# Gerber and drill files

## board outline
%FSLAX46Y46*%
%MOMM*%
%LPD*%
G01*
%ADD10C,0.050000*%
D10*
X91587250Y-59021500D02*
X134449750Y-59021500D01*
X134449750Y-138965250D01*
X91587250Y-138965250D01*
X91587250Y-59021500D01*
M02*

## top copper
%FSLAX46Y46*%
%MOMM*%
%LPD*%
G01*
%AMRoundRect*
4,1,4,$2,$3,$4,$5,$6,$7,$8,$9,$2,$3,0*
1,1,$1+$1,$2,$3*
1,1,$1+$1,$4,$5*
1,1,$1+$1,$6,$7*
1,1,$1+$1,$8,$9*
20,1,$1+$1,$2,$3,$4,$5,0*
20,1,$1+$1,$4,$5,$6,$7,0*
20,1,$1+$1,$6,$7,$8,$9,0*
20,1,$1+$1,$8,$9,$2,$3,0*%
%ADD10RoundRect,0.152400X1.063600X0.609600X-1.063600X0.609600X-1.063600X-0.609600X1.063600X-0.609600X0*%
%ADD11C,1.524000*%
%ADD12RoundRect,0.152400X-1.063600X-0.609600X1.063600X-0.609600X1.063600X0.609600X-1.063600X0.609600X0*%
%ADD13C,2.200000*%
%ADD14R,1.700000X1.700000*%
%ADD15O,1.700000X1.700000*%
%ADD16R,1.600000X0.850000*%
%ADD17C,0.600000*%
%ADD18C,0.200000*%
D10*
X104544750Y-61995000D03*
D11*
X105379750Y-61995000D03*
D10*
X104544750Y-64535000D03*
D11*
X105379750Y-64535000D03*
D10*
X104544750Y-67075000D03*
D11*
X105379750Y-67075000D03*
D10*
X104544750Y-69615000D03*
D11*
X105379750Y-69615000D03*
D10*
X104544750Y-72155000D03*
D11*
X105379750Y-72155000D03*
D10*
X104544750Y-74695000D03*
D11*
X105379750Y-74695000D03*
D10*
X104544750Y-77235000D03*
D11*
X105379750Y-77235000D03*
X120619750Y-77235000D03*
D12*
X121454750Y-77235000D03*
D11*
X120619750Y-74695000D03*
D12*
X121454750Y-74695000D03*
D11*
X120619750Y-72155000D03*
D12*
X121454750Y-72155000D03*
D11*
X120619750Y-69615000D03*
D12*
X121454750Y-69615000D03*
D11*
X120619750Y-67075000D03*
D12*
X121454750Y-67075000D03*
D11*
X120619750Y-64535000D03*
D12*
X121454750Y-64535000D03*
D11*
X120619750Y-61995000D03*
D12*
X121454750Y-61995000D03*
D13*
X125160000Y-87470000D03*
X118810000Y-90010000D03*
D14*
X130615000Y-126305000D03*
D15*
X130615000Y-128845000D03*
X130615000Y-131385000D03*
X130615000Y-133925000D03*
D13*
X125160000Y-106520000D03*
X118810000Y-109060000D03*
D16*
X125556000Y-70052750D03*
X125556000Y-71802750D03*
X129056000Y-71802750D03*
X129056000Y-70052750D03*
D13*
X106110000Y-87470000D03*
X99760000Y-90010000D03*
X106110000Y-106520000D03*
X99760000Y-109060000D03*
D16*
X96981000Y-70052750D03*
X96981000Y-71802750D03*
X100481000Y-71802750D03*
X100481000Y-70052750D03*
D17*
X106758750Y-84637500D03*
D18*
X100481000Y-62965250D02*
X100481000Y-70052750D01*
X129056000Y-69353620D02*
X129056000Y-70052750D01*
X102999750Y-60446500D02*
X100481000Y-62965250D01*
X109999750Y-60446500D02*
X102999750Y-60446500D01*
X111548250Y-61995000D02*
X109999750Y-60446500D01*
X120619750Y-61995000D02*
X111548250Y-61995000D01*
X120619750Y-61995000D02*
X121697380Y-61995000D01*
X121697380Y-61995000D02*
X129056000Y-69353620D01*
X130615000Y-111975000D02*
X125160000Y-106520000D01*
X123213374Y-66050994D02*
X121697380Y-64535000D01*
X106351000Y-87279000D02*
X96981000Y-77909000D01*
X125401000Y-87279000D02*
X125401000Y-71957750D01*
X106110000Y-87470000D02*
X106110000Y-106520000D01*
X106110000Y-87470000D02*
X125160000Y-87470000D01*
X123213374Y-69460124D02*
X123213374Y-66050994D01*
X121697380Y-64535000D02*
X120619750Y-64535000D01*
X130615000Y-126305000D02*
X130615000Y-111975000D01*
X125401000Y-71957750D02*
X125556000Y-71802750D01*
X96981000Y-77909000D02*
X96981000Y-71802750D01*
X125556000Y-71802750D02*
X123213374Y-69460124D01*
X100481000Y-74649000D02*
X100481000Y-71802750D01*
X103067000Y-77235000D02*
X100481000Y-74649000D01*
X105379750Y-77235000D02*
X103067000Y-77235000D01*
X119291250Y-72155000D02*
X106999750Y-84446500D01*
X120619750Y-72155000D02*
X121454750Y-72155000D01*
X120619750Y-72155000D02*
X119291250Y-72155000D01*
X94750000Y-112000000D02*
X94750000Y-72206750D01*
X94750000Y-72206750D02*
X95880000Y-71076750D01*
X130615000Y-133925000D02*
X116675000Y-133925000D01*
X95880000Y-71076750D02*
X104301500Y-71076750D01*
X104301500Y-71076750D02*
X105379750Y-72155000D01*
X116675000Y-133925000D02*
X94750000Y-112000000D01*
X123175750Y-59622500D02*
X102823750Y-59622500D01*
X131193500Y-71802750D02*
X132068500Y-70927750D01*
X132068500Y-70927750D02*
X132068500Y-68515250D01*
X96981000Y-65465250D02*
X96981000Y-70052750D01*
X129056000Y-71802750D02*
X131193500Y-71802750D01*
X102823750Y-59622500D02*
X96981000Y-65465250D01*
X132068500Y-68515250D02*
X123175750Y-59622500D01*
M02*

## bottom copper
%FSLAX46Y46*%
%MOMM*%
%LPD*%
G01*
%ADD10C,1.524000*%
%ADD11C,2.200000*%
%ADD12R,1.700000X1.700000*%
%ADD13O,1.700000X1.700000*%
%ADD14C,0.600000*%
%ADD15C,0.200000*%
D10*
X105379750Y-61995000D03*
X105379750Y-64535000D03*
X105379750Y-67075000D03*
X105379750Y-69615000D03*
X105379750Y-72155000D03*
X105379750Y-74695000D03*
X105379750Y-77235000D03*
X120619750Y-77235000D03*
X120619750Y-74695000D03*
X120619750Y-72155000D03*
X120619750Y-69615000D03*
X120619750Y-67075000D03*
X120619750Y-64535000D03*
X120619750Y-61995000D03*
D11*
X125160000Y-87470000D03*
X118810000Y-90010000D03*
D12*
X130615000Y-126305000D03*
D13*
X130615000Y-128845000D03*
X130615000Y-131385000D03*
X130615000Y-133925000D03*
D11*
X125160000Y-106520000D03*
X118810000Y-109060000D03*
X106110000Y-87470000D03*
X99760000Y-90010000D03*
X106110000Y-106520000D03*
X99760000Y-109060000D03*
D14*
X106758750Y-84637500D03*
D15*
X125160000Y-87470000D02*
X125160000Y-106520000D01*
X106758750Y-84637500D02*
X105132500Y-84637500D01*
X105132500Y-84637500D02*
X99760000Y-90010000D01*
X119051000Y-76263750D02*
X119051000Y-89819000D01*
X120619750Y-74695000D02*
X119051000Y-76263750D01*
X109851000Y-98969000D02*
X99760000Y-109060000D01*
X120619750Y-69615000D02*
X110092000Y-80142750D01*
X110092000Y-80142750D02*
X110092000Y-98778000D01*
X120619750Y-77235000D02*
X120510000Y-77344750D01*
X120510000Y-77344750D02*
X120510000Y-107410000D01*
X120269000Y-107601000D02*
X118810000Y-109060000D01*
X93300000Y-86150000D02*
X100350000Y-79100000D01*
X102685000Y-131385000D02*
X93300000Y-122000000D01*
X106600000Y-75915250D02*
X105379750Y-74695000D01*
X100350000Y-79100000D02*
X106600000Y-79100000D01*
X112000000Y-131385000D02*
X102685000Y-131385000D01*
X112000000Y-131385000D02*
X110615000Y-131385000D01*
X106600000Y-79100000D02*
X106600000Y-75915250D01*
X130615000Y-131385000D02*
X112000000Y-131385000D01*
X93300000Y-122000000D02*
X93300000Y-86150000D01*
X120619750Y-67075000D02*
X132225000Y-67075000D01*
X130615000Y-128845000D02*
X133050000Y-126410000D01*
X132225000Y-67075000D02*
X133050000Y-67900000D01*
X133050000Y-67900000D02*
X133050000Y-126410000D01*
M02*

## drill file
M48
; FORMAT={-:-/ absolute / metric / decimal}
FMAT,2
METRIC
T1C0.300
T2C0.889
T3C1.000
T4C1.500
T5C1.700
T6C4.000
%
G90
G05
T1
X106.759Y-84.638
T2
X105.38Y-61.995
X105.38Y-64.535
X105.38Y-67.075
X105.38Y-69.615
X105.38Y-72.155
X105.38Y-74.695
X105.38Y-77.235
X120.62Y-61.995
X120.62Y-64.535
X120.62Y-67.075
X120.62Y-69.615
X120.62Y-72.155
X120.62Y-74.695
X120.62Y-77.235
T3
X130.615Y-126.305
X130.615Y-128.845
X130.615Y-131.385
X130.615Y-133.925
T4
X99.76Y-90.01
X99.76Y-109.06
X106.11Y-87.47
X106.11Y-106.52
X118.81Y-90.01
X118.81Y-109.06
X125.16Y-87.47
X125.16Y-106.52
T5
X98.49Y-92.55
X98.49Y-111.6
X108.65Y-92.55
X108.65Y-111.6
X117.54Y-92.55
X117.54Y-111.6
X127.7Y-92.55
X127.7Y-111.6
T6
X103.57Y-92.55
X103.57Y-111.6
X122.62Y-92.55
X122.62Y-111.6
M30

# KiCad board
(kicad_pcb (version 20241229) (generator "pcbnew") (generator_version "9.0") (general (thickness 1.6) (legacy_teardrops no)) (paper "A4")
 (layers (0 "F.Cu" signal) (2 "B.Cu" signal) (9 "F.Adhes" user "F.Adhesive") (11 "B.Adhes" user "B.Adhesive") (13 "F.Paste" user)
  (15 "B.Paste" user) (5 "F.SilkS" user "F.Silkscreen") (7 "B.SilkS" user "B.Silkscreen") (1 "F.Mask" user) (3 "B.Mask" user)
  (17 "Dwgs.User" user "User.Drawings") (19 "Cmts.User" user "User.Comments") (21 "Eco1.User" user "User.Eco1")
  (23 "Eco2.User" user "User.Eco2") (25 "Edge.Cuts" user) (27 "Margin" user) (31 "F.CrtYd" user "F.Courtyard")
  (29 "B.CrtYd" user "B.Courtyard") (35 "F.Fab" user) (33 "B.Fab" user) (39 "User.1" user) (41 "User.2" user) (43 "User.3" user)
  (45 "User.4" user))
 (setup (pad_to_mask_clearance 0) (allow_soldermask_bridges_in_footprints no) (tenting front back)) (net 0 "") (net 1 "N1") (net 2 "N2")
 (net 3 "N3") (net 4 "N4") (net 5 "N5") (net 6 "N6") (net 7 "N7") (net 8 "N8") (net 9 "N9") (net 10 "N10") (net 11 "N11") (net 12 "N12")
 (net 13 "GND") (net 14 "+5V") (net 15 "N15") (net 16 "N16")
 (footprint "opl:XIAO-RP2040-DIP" (layer "F.Cu") (at 112.99975 69.615)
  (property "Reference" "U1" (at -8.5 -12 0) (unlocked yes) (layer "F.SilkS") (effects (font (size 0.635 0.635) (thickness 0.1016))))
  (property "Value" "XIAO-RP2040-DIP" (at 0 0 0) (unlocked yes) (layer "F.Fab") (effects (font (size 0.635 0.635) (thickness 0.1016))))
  (pad "1" smd roundrect (at -8.455 -7.62 180) (size 2.432 1.524) (layers "F.Cu" "F.Mask") (roundrect_rratio 0.1) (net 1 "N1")
   (thermal_bridge_angle 45))
  (pad "1" thru_hole circle (at -7.62 -7.62 180) (size 1.524 1.524) (drill 0.889) (layers "*.Cu" "*.Mask") (remove_unused_layers no)
   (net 1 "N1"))
  (pad "2" smd roundrect (at -8.455 -5.08 180) (size 2.432 1.524) (layers "F.Cu" "F.Mask") (roundrect_rratio 0.1) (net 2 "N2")
   (thermal_bridge_angle 45))
  (pad "2" thru_hole circle (at -7.62 -5.08 180) (size 1.524 1.524) (drill 0.889) (layers "*.Cu" "*.Mask") (remove_unused_layers no)
   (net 2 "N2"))
  (pad "3" smd roundrect (at -8.455 -2.54 180) (size 2.432 1.524) (layers "F.Cu" "F.Mask") (roundrect_rratio 0.1) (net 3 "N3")
   (thermal_bridge_angle 45))
  (pad "3" thru_hole circle (at -7.62 -2.54 180) (size 1.524 1.524) (drill 0.889) (layers "*.Cu" "*.Mask") (remove_unused_layers no)
   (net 3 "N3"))
  (pad "4" smd roundrect (at -8.455 0 180) (size 2.432 1.524) (layers "F.Cu" "F.Mask") (roundrect_rratio 0.1) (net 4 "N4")
   (thermal_bridge_angle 45))
  (pad "4" thru_hole circle (at -7.62 0 180) (size 1.524 1.524) (drill 0.889) (layers "*.Cu" "*.Mask") (remove_unused_layers no)
   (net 4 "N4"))
  (pad "5" smd roundrect (at -8.455 2.54 180) (size 2.432 1.524) (layers "F.Cu" "F.Mask") (roundrect_rratio 0.1) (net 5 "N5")
   (thermal_bridge_angle 45))
  (pad "5" thru_hole circle (at -7.62 2.54 180) (size 1.524 1.524) (drill 0.889) (layers "*.Cu" "*.Mask") (remove_unused_layers no)
   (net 5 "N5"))
  (pad "6" smd roundrect (at -8.455 5.08 180) (size 2.432 1.524) (layers "F.Cu" "F.Mask") (roundrect_rratio 0.1) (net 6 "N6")
   (thermal_bridge_angle 45))
  (pad "6" thru_hole circle (at -7.62 5.08 180) (size 1.524 1.524) (drill 0.889) (layers "*.Cu" "*.Mask") (remove_unused_layers no)
   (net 6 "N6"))
  (pad "7" smd roundrect (at -8.455 7.62 180) (size 2.432 1.524) (layers "F.Cu" "F.Mask") (roundrect_rratio 0.1) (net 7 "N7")
   (thermal_bridge_angle 45))
  (pad "7" thru_hole circle (at -7.62 7.62 180) (size 1.524 1.524) (drill 0.889) (layers "*.Cu" "*.Mask") (remove_unused_layers no)
   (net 7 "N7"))
  (pad "8" thru_hole circle (at 7.62 7.62) (size 1.524 1.524) (drill 0.889) (layers "*.Cu" "*.Mask") (remove_unused_layers no) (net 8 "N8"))
  (pad "8" smd roundrect (at 8.455 7.62) (size 2.432 1.524) (layers "F.Cu" "F.Mask") (roundrect_rratio 0.1) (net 8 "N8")
   (thermal_bridge_angle 45))
  (pad "9" thru_hole circle (at 7.62 5.08) (size 1.524 1.524) (drill 0.889) (layers "*.Cu" "*.Mask") (remove_unused_layers no) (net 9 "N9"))
  (pad "9" smd roundrect (at 8.455 5.08) (size 2.432 1.524) (layers "F.Cu" "F.Mask") (roundrect_rratio 0.1) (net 9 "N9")
   (thermal_bridge_angle 45))
  (pad "10" thru_hole circle (at 7.62 2.54) (size 1.524 1.524) (drill 0.889) (layers "*.Cu" "*.Mask") (remove_unused_layers no)
   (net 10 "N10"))
  (pad "10" smd roundrect (at 8.455 2.54) (size 2.432 1.524) (layers "F.Cu" "F.Mask") (roundrect_rratio 0.1) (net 10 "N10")
   (thermal_bridge_angle 45))
  (pad "11" thru_hole circle (at 7.62 0) (size 1.524 1.524) (drill 0.889) (layers "*.Cu" "*.Mask") (remove_unused_layers no) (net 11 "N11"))
  (pad "11" smd roundrect (at 8.455 0) (size 2.432 1.524) (layers "F.Cu" "F.Mask") (roundrect_rratio 0.1) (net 11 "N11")
   (thermal_bridge_angle 45))
  (pad "12" thru_hole circle (at 7.62 -2.54) (size 1.524 1.524) (drill 0.889) (layers "*.Cu" "*.Mask") (remove_unused_layers no)
   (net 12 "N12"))
  (pad "12" smd roundrect (at 8.455 -2.54) (size 2.432 1.524) (layers "F.Cu" "F.Mask") (roundrect_rratio 0.1) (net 12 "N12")
   (thermal_bridge_angle 45))
  (pad "13" thru_hole circle (at 7.62 -5.08) (size 1.524 1.524) (drill 0.889) (layers "*.Cu" "*.Mask") (remove_unused_layers no)
   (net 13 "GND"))
  (pad "13" smd roundrect (at 8.455 -5.08) (size 2.432 1.524) (layers "F.Cu" "F.Mask") (roundrect_rratio 0.1) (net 13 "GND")
   (thermal_bridge_angle 45))
  (pad "14" thru_hole circle (at 7.62 -7.62) (size 1.524 1.524) (drill 0.889) (layers "*.Cu" "*.Mask") (remove_unused_layers no)
   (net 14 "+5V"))
  (pad "14" smd roundrect (at 8.455 -7.62) (size 2.432 1.524) (layers "F.Cu" "F.Mask") (roundrect_rratio 0.1) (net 14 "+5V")
   (thermal_bridge_angle 45)))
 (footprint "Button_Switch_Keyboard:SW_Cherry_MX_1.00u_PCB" (layer "F.Cu") (at 125.16 87.47)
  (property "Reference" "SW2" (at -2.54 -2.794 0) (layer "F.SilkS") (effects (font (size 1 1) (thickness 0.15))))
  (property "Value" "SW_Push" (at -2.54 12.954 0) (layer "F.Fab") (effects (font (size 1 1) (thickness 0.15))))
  (pad "" np_thru_hole circle (at -7.62 5.08) (size 1.7 1.7) (drill 1.7) (layers "*.Cu" "*.Mask"))
  (pad "" np_thru_hole circle (at -2.54 5.08) (size 4 4) (drill 4) (layers "*.Cu" "*.Mask"))
  (pad "" np_thru_hole circle (at 2.54 5.08) (size 1.7 1.7) (drill 1.7) (layers "*.Cu" "*.Mask"))
  (pad "1" thru_hole circle (at 0 0) (size 2.2 2.2) (drill 1.5) (layers "*.Cu" "*.Mask") (remove_unused_layers no) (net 13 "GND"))
  (pad "2" thru_hole circle (at -6.35 2.54) (size 2.2 2.2) (drill 1.5) (layers "*.Cu" "*.Mask") (remove_unused_layers no) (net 9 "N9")))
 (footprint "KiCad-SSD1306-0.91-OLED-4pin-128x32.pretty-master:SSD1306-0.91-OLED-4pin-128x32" (layer "F.Cu") (at 94.115 124.115)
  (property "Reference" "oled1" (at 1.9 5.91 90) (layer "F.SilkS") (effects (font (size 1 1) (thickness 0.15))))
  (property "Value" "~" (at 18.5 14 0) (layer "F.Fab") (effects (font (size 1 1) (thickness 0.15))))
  (pad "1" thru_hole rect (at 36.5 2.19) (size 1.7 1.7) (drill 1) (layers "*.Cu" "*.Mask") (remove_unused_layers no) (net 13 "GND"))
  (pad "2" thru_hole oval (at 36.5 4.73) (size 1.7 1.7) (drill 1) (layers "*.Cu" "*.Mask") (remove_unused_layers no) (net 12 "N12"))
  (pad "3" thru_hole oval (at 36.5 7.27) (size 1.7 1.7) (drill 1) (layers "*.Cu" "*.Mask") (remove_unused_layers no) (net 6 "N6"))
  (pad "4" thru_hole oval (at 36.5 9.81) (size 1.7 1.7) (drill 1) (layers "*.Cu" "*.Mask") (remove_unused_layers no) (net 5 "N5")))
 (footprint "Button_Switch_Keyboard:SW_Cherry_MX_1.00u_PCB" (layer "F.Cu") (at 125.16 106.52)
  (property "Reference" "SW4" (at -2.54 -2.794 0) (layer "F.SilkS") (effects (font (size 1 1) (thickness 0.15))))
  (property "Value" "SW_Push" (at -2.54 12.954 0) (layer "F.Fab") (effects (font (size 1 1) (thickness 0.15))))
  (pad "" np_thru_hole circle (at -7.62 5.08) (size 1.7 1.7) (drill 1.7) (layers "*.Cu" "*.Mask"))
  (pad "" np_thru_hole circle (at -2.54 5.08) (size 4 4) (drill 4) (layers "*.Cu" "*.Mask"))
  (pad "" np_thru_hole circle (at 2.54 5.08) (size 1.7 1.7) (drill 1.7) (layers "*.Cu" "*.Mask"))
  (pad "1" thru_hole circle (at 0 0) (size 2.2 2.2) (drill 1.5) (layers "*.Cu" "*.Mask") (remove_unused_layers no) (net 13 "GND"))
  (pad "2" thru_hole circle (at -6.35 2.54) (size 2.2 2.2) (drill 1.5) (layers "*.Cu" "*.Mask") (remove_unused_layers no) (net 8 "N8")))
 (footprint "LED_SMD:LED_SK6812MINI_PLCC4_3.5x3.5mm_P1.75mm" (layer "F.Cu") (at 127.306 70.92775)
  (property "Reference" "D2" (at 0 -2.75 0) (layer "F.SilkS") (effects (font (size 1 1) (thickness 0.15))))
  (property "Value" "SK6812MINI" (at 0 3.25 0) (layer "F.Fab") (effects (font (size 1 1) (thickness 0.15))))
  (pad "1" smd rect (at -1.75 -0.875) (size 1.6 0.85) (layers "F.Cu" "F.Mask" "F.Paste") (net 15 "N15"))
  (pad "2" smd rect (at -1.75 0.875) (size 1.6 0.85) (layers "F.Cu" "F.Mask" "F.Paste") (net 13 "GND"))
  (pad "3" smd rect (at 1.75 0.875) (size 1.6 0.85) (layers "F.Cu" "F.Mask" "F.Paste") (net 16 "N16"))
  (pad "4" smd rect (at 1.75 -0.875) (size 1.6 0.85) (layers "F.Cu" "F.Mask" "F.Paste") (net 14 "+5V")))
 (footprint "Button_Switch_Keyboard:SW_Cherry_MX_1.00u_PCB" (layer "F.Cu") (at 106.11 87.47)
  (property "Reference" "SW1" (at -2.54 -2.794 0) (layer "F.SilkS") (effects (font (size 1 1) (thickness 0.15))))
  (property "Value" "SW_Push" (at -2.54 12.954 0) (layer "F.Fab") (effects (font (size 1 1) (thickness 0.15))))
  (pad "" np_thru_hole circle (at -7.62 5.08) (size 1.7 1.7) (drill 1.7) (layers "*.Cu" "*.Mask"))
  (pad "" np_thru_hole circle (at -2.54 5.08) (size 4 4) (drill 4) (layers "*.Cu" "*.Mask"))
  (pad "" np_thru_hole circle (at 2.54 5.08) (size 1.7 1.7) (drill 1.7) (layers "*.Cu" "*.Mask"))
  (pad "1" thru_hole circle (at 0 0) (size 2.2 2.2) (drill 1.5) (layers "*.Cu" "*.Mask") (remove_unused_layers no) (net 13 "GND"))
  (pad "2" thru_hole circle (at -6.35 2.54) (size 2.2 2.2) (drill 1.5) (layers "*.Cu" "*.Mask") (remove_unused_layers no) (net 10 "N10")))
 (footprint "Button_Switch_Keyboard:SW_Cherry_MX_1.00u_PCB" (layer "F.Cu") (at 106.11 106.52)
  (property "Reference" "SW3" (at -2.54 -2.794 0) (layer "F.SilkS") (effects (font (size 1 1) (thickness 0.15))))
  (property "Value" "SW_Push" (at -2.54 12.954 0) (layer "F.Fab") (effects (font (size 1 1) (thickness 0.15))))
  (pad "" np_thru_hole circle (at -7.62 5.08) (size 1.7 1.7) (drill 1.7) (layers "*.Cu" "*.Mask"))
  (pad "" np_thru_hole circle (at -2.54 5.08) (size 4 4) (drill 4) (layers "*.Cu" "*.Mask"))
  (pad "" np_thru_hole circle (at 2.54 5.08) (size 1.7 1.7) (drill 1.7) (layers "*.Cu" "*.Mask"))
  (pad "1" thru_hole circle (at 0 0) (size 2.2 2.2) (drill 1.5) (layers "*.Cu" "*.Mask") (remove_unused_layers no) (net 13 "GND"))
  (pad "2" thru_hole circle (at -6.35 2.54) (size 2.2 2.2) (drill 1.5) (layers "*.Cu" "*.Mask") (remove_unused_layers no) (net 11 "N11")))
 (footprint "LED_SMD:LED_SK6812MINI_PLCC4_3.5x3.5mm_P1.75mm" (layer "F.Cu") (at 98.731 70.92775)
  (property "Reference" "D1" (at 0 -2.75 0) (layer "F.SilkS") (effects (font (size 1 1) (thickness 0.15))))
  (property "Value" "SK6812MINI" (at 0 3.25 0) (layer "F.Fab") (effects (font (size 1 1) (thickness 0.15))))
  (pad "1" smd rect (at -1.75 -0.875) (size 1.6 0.85) (layers "F.Cu" "F.Mask" "F.Paste") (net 16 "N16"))
  (pad "2" smd rect (at -1.75 0.875) (size 1.6 0.85) (layers "F.Cu" "F.Mask" "F.Paste") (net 13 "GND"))
  (pad "3" smd rect (at 1.75 0.875) (size 1.6 0.85) (layers "F.Cu" "F.Mask" "F.Paste") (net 7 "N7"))
  (pad "4" smd rect (at 1.75 -0.875) (size 1.6 0.85) (layers "F.Cu" "F.Mask" "F.Paste") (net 14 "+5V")))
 (gr_rect (start 91.58725 59.0215) (end 134.44975 138.96525) (stroke (width 0.05) (type default)) (fill no) (layer "Edge.Cuts"))
 (segment (start 100.481 62.96525) (end 100.481 70.05275) (width 0.2) (layer "F.Cu") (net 14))
 (segment (start 129.056 69.35362) (end 129.056 70.05275) (width 0.2) (layer "F.Cu") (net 14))
 (segment (start 102.99975 60.4465) (end 100.481 62.96525) (width 0.2) (layer "F.Cu") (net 14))
 (segment (start 109.99975 60.4465) (end 102.99975 60.4465) (width 0.2) (layer "F.Cu") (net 14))
 (segment (start 111.54825 61.995) (end 109.99975 60.4465) (width 0.2) (layer "F.Cu") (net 14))
 (segment (start 120.61975 61.995) (end 111.54825 61.995) (width 0.2) (layer "F.Cu") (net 14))
 (segment (start 120.61975 61.995) (end 121.69738 61.995) (width 0.2) (layer "F.Cu") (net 14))
 (segment (start 121.69738 61.995) (end 129.056 69.35362) (width 0.2) (layer "F.Cu") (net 14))
 (segment (start 130.615 111.975) (end 125.16 106.52) (width 0.2) (layer "F.Cu") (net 13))
 (segment (start 123.213374 66.050994) (end 121.69738 64.535) (width 0.2) (layer "F.Cu") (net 13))
 (segment (start 106.351 87.279) (end 96.981 77.909) (width 0.2) (layer "F.Cu") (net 13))
 (segment (start 125.401 87.279) (end 125.401 71.95775) (width 0.2) (layer "F.Cu") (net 13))
 (segment (start 106.11 87.47) (end 106.11 106.52) (width 0.2) (layer "F.Cu") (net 13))
 (segment (start 106.11 87.47) (end 125.16 87.47) (width 0.2) (layer "F.Cu") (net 13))
 (segment (start 123.213374 69.460124) (end 123.213374 66.050994) (width 0.2) (layer "F.Cu") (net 13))
 (segment (start 121.69738 64.535) (end 120.61975 64.535) (width 0.2) (layer "F.Cu") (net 13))
 (segment (start 130.615 126.305) (end 130.615 111.975) (width 0.2) (layer "F.Cu") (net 13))
 (segment (start 125.401 71.95775) (end 125.556 71.80275) (width 0.2) (layer "F.Cu") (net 13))
 (segment (start 96.981 77.909) (end 96.981 71.80275) (width 0.2) (layer "F.Cu") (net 13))
 (segment (start 125.556 71.80275) (end 123.213374 69.460124) (width 0.2) (layer "F.Cu") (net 13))
 (segment (start 125.16 87.47) (end 125.16 106.52) (width 0.2) (layer "B.Cu") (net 13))
 (segment (start 100.481 74.649) (end 100.481 71.80275) (width 0.2) (layer "F.Cu") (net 7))
 (segment (start 103.067 77.235) (end 100.481 74.649) (width 0.2) (layer "F.Cu") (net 7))
 (segment (start 105.37975 77.235) (end 103.067 77.235) (width 0.2) (layer "F.Cu") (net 7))
 (segment (start 119.29125 72.155) (end 106.99975 84.4465) (width 0.2) (layer "F.Cu") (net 10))
 (segment (start 120.61975 72.155) (end 121.45475 72.155) (width 0.2) (layer "F.Cu") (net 10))
 (segment (start 120.61975 72.155) (end 119.29125 72.155) (width 0.2) (layer "F.Cu") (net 10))
 (via (at 106.75875 84.6375) (size 0.6) (drill 0.3) (layers "F.Cu" "B.Cu") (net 10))
 (segment (start 106.75875 84.6375) (end 105.1325 84.6375) (width 0.2) (layer "B.Cu") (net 10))
 (segment (start 105.1325 84.6375) (end 99.76 90.01) (width 0.2) (layer "B.Cu") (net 10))
 (segment (start 119.051 76.26375) (end 119.051 89.819) (width 0.2) (layer "B.Cu") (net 9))
 (segment (start 120.61975 74.695) (end 119.051 76.26375) (width 0.2) (layer "B.Cu") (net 9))
 (segment (start 109.851 98.969) (end 99.76 109.06) (width 0.2) (layer "B.Cu") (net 11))
 (segment (start 120.61975 69.615) (end 110.092 80.14275) (width 0.2) (layer "B.Cu") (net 11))
 (segment (start 110.092 80.14275) (end 110.092 98.778) (width 0.2) (layer "B.Cu") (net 11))
 (segment (start 120.61975 77.235) (end 120.51 77.34475) (width 0.2) (layer "B.Cu") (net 8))
 (segment (start 120.51 77.34475) (end 120.51 107.41) (width 0.2) (layer "B.Cu") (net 8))
 (segment (start 120.269 107.601) (end 118.81 109.06) (width 0.2) (layer "B.Cu") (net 8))
 (segment (start 93.3 86.15) (end 100.35 79.1) (width 0.2) (layer "B.Cu") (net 6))
 (segment (start 102.685 131.385) (end 93.3 122) (width 0.2) (layer "B.Cu") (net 6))
 (segment (start 106.6 75.91525) (end 105.37975 74.695) (width 0.2) (layer "B.Cu") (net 6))
 (segment (start 100.35 79.1) (end 106.6 79.1) (width 0.2) (layer "B.Cu") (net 6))
 (segment (start 112 131.385) (end 102.685 131.385) (width 0.2) (layer "B.Cu") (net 6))
 (segment (start 112 131.385) (end 110.615 131.385) (width 0.2) (layer "B.Cu") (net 6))
 (segment (start 106.6 79.1) (end 106.6 75.91525) (width 0.2) (layer "B.Cu") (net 6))
 (segment (start 130.615 131.385) (end 112 131.385) (width 0.2) (layer "B.Cu") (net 6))
 (segment (start 93.3 122) (end 93.3 86.15) (width 0.2) (layer "B.Cu") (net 6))
 (segment (start 94.75 112) (end 94.75 72.20675) (width 0.2) (layer "F.Cu") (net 5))
 (segment (start 94.75 72.20675) (end 95.88 71.07675) (width 0.2) (layer "F.Cu") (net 5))
 (segment (start 130.615 133.925) (end 116.675 133.925) (width 0.2) (layer "F.Cu") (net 5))
 (segment (start 95.88 71.07675) (end 104.3015 71.07675) (width 0.2) (layer "F.Cu") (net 5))
 (segment (start 104.3015 71.07675) (end 105.37975 72.155) (width 0.2) (layer "F.Cu") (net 5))
 (segment (start 116.675 133.925) (end 94.75 112) (width 0.2) (layer "F.Cu") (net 5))
 (segment (start 123.17575 59.6225) (end 102.82375 59.6225) (width 0.2) (layer "F.Cu") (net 16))
 (segment (start 131.1935 71.80275) (end 132.0685 70.92775) (width 0.2) (layer "F.Cu") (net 16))
 (segment (start 132.0685 70.92775) (end 132.0685 68.51525) (width 0.2) (layer "F.Cu") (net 16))
 (segment (start 96.981 65.46525) (end 96.981 70.05275) (width 0.2) (layer "F.Cu") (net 16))
 (segment (start 129.056 71.80275) (end 131.1935 71.80275) (width 0.2) (layer "F.Cu") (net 16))
 (segment (start 102.82375 59.6225) (end 96.981 65.46525) (width 0.2) (layer "F.Cu") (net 16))
 (segment (start 132.0685 68.51525) (end 123.17575 59.6225) (width 0.2) (layer "F.Cu") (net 16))
 (segment (start 120.61975 67.075) (end 132.225 67.075) (width 0.2) (layer "B.Cu") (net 12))
 (segment (start 130.615 128.845) (end 133.05 126.41) (width 0.2) (layer "B.Cu") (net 12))
 (segment (start 132.225 67.075) (end 133.05 67.9) (width 0.2) (layer "B.Cu") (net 12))
 (segment (start 133.05 67.9) (end 133.05 126.41) (width 0.2) (layer "B.Cu") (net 12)))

